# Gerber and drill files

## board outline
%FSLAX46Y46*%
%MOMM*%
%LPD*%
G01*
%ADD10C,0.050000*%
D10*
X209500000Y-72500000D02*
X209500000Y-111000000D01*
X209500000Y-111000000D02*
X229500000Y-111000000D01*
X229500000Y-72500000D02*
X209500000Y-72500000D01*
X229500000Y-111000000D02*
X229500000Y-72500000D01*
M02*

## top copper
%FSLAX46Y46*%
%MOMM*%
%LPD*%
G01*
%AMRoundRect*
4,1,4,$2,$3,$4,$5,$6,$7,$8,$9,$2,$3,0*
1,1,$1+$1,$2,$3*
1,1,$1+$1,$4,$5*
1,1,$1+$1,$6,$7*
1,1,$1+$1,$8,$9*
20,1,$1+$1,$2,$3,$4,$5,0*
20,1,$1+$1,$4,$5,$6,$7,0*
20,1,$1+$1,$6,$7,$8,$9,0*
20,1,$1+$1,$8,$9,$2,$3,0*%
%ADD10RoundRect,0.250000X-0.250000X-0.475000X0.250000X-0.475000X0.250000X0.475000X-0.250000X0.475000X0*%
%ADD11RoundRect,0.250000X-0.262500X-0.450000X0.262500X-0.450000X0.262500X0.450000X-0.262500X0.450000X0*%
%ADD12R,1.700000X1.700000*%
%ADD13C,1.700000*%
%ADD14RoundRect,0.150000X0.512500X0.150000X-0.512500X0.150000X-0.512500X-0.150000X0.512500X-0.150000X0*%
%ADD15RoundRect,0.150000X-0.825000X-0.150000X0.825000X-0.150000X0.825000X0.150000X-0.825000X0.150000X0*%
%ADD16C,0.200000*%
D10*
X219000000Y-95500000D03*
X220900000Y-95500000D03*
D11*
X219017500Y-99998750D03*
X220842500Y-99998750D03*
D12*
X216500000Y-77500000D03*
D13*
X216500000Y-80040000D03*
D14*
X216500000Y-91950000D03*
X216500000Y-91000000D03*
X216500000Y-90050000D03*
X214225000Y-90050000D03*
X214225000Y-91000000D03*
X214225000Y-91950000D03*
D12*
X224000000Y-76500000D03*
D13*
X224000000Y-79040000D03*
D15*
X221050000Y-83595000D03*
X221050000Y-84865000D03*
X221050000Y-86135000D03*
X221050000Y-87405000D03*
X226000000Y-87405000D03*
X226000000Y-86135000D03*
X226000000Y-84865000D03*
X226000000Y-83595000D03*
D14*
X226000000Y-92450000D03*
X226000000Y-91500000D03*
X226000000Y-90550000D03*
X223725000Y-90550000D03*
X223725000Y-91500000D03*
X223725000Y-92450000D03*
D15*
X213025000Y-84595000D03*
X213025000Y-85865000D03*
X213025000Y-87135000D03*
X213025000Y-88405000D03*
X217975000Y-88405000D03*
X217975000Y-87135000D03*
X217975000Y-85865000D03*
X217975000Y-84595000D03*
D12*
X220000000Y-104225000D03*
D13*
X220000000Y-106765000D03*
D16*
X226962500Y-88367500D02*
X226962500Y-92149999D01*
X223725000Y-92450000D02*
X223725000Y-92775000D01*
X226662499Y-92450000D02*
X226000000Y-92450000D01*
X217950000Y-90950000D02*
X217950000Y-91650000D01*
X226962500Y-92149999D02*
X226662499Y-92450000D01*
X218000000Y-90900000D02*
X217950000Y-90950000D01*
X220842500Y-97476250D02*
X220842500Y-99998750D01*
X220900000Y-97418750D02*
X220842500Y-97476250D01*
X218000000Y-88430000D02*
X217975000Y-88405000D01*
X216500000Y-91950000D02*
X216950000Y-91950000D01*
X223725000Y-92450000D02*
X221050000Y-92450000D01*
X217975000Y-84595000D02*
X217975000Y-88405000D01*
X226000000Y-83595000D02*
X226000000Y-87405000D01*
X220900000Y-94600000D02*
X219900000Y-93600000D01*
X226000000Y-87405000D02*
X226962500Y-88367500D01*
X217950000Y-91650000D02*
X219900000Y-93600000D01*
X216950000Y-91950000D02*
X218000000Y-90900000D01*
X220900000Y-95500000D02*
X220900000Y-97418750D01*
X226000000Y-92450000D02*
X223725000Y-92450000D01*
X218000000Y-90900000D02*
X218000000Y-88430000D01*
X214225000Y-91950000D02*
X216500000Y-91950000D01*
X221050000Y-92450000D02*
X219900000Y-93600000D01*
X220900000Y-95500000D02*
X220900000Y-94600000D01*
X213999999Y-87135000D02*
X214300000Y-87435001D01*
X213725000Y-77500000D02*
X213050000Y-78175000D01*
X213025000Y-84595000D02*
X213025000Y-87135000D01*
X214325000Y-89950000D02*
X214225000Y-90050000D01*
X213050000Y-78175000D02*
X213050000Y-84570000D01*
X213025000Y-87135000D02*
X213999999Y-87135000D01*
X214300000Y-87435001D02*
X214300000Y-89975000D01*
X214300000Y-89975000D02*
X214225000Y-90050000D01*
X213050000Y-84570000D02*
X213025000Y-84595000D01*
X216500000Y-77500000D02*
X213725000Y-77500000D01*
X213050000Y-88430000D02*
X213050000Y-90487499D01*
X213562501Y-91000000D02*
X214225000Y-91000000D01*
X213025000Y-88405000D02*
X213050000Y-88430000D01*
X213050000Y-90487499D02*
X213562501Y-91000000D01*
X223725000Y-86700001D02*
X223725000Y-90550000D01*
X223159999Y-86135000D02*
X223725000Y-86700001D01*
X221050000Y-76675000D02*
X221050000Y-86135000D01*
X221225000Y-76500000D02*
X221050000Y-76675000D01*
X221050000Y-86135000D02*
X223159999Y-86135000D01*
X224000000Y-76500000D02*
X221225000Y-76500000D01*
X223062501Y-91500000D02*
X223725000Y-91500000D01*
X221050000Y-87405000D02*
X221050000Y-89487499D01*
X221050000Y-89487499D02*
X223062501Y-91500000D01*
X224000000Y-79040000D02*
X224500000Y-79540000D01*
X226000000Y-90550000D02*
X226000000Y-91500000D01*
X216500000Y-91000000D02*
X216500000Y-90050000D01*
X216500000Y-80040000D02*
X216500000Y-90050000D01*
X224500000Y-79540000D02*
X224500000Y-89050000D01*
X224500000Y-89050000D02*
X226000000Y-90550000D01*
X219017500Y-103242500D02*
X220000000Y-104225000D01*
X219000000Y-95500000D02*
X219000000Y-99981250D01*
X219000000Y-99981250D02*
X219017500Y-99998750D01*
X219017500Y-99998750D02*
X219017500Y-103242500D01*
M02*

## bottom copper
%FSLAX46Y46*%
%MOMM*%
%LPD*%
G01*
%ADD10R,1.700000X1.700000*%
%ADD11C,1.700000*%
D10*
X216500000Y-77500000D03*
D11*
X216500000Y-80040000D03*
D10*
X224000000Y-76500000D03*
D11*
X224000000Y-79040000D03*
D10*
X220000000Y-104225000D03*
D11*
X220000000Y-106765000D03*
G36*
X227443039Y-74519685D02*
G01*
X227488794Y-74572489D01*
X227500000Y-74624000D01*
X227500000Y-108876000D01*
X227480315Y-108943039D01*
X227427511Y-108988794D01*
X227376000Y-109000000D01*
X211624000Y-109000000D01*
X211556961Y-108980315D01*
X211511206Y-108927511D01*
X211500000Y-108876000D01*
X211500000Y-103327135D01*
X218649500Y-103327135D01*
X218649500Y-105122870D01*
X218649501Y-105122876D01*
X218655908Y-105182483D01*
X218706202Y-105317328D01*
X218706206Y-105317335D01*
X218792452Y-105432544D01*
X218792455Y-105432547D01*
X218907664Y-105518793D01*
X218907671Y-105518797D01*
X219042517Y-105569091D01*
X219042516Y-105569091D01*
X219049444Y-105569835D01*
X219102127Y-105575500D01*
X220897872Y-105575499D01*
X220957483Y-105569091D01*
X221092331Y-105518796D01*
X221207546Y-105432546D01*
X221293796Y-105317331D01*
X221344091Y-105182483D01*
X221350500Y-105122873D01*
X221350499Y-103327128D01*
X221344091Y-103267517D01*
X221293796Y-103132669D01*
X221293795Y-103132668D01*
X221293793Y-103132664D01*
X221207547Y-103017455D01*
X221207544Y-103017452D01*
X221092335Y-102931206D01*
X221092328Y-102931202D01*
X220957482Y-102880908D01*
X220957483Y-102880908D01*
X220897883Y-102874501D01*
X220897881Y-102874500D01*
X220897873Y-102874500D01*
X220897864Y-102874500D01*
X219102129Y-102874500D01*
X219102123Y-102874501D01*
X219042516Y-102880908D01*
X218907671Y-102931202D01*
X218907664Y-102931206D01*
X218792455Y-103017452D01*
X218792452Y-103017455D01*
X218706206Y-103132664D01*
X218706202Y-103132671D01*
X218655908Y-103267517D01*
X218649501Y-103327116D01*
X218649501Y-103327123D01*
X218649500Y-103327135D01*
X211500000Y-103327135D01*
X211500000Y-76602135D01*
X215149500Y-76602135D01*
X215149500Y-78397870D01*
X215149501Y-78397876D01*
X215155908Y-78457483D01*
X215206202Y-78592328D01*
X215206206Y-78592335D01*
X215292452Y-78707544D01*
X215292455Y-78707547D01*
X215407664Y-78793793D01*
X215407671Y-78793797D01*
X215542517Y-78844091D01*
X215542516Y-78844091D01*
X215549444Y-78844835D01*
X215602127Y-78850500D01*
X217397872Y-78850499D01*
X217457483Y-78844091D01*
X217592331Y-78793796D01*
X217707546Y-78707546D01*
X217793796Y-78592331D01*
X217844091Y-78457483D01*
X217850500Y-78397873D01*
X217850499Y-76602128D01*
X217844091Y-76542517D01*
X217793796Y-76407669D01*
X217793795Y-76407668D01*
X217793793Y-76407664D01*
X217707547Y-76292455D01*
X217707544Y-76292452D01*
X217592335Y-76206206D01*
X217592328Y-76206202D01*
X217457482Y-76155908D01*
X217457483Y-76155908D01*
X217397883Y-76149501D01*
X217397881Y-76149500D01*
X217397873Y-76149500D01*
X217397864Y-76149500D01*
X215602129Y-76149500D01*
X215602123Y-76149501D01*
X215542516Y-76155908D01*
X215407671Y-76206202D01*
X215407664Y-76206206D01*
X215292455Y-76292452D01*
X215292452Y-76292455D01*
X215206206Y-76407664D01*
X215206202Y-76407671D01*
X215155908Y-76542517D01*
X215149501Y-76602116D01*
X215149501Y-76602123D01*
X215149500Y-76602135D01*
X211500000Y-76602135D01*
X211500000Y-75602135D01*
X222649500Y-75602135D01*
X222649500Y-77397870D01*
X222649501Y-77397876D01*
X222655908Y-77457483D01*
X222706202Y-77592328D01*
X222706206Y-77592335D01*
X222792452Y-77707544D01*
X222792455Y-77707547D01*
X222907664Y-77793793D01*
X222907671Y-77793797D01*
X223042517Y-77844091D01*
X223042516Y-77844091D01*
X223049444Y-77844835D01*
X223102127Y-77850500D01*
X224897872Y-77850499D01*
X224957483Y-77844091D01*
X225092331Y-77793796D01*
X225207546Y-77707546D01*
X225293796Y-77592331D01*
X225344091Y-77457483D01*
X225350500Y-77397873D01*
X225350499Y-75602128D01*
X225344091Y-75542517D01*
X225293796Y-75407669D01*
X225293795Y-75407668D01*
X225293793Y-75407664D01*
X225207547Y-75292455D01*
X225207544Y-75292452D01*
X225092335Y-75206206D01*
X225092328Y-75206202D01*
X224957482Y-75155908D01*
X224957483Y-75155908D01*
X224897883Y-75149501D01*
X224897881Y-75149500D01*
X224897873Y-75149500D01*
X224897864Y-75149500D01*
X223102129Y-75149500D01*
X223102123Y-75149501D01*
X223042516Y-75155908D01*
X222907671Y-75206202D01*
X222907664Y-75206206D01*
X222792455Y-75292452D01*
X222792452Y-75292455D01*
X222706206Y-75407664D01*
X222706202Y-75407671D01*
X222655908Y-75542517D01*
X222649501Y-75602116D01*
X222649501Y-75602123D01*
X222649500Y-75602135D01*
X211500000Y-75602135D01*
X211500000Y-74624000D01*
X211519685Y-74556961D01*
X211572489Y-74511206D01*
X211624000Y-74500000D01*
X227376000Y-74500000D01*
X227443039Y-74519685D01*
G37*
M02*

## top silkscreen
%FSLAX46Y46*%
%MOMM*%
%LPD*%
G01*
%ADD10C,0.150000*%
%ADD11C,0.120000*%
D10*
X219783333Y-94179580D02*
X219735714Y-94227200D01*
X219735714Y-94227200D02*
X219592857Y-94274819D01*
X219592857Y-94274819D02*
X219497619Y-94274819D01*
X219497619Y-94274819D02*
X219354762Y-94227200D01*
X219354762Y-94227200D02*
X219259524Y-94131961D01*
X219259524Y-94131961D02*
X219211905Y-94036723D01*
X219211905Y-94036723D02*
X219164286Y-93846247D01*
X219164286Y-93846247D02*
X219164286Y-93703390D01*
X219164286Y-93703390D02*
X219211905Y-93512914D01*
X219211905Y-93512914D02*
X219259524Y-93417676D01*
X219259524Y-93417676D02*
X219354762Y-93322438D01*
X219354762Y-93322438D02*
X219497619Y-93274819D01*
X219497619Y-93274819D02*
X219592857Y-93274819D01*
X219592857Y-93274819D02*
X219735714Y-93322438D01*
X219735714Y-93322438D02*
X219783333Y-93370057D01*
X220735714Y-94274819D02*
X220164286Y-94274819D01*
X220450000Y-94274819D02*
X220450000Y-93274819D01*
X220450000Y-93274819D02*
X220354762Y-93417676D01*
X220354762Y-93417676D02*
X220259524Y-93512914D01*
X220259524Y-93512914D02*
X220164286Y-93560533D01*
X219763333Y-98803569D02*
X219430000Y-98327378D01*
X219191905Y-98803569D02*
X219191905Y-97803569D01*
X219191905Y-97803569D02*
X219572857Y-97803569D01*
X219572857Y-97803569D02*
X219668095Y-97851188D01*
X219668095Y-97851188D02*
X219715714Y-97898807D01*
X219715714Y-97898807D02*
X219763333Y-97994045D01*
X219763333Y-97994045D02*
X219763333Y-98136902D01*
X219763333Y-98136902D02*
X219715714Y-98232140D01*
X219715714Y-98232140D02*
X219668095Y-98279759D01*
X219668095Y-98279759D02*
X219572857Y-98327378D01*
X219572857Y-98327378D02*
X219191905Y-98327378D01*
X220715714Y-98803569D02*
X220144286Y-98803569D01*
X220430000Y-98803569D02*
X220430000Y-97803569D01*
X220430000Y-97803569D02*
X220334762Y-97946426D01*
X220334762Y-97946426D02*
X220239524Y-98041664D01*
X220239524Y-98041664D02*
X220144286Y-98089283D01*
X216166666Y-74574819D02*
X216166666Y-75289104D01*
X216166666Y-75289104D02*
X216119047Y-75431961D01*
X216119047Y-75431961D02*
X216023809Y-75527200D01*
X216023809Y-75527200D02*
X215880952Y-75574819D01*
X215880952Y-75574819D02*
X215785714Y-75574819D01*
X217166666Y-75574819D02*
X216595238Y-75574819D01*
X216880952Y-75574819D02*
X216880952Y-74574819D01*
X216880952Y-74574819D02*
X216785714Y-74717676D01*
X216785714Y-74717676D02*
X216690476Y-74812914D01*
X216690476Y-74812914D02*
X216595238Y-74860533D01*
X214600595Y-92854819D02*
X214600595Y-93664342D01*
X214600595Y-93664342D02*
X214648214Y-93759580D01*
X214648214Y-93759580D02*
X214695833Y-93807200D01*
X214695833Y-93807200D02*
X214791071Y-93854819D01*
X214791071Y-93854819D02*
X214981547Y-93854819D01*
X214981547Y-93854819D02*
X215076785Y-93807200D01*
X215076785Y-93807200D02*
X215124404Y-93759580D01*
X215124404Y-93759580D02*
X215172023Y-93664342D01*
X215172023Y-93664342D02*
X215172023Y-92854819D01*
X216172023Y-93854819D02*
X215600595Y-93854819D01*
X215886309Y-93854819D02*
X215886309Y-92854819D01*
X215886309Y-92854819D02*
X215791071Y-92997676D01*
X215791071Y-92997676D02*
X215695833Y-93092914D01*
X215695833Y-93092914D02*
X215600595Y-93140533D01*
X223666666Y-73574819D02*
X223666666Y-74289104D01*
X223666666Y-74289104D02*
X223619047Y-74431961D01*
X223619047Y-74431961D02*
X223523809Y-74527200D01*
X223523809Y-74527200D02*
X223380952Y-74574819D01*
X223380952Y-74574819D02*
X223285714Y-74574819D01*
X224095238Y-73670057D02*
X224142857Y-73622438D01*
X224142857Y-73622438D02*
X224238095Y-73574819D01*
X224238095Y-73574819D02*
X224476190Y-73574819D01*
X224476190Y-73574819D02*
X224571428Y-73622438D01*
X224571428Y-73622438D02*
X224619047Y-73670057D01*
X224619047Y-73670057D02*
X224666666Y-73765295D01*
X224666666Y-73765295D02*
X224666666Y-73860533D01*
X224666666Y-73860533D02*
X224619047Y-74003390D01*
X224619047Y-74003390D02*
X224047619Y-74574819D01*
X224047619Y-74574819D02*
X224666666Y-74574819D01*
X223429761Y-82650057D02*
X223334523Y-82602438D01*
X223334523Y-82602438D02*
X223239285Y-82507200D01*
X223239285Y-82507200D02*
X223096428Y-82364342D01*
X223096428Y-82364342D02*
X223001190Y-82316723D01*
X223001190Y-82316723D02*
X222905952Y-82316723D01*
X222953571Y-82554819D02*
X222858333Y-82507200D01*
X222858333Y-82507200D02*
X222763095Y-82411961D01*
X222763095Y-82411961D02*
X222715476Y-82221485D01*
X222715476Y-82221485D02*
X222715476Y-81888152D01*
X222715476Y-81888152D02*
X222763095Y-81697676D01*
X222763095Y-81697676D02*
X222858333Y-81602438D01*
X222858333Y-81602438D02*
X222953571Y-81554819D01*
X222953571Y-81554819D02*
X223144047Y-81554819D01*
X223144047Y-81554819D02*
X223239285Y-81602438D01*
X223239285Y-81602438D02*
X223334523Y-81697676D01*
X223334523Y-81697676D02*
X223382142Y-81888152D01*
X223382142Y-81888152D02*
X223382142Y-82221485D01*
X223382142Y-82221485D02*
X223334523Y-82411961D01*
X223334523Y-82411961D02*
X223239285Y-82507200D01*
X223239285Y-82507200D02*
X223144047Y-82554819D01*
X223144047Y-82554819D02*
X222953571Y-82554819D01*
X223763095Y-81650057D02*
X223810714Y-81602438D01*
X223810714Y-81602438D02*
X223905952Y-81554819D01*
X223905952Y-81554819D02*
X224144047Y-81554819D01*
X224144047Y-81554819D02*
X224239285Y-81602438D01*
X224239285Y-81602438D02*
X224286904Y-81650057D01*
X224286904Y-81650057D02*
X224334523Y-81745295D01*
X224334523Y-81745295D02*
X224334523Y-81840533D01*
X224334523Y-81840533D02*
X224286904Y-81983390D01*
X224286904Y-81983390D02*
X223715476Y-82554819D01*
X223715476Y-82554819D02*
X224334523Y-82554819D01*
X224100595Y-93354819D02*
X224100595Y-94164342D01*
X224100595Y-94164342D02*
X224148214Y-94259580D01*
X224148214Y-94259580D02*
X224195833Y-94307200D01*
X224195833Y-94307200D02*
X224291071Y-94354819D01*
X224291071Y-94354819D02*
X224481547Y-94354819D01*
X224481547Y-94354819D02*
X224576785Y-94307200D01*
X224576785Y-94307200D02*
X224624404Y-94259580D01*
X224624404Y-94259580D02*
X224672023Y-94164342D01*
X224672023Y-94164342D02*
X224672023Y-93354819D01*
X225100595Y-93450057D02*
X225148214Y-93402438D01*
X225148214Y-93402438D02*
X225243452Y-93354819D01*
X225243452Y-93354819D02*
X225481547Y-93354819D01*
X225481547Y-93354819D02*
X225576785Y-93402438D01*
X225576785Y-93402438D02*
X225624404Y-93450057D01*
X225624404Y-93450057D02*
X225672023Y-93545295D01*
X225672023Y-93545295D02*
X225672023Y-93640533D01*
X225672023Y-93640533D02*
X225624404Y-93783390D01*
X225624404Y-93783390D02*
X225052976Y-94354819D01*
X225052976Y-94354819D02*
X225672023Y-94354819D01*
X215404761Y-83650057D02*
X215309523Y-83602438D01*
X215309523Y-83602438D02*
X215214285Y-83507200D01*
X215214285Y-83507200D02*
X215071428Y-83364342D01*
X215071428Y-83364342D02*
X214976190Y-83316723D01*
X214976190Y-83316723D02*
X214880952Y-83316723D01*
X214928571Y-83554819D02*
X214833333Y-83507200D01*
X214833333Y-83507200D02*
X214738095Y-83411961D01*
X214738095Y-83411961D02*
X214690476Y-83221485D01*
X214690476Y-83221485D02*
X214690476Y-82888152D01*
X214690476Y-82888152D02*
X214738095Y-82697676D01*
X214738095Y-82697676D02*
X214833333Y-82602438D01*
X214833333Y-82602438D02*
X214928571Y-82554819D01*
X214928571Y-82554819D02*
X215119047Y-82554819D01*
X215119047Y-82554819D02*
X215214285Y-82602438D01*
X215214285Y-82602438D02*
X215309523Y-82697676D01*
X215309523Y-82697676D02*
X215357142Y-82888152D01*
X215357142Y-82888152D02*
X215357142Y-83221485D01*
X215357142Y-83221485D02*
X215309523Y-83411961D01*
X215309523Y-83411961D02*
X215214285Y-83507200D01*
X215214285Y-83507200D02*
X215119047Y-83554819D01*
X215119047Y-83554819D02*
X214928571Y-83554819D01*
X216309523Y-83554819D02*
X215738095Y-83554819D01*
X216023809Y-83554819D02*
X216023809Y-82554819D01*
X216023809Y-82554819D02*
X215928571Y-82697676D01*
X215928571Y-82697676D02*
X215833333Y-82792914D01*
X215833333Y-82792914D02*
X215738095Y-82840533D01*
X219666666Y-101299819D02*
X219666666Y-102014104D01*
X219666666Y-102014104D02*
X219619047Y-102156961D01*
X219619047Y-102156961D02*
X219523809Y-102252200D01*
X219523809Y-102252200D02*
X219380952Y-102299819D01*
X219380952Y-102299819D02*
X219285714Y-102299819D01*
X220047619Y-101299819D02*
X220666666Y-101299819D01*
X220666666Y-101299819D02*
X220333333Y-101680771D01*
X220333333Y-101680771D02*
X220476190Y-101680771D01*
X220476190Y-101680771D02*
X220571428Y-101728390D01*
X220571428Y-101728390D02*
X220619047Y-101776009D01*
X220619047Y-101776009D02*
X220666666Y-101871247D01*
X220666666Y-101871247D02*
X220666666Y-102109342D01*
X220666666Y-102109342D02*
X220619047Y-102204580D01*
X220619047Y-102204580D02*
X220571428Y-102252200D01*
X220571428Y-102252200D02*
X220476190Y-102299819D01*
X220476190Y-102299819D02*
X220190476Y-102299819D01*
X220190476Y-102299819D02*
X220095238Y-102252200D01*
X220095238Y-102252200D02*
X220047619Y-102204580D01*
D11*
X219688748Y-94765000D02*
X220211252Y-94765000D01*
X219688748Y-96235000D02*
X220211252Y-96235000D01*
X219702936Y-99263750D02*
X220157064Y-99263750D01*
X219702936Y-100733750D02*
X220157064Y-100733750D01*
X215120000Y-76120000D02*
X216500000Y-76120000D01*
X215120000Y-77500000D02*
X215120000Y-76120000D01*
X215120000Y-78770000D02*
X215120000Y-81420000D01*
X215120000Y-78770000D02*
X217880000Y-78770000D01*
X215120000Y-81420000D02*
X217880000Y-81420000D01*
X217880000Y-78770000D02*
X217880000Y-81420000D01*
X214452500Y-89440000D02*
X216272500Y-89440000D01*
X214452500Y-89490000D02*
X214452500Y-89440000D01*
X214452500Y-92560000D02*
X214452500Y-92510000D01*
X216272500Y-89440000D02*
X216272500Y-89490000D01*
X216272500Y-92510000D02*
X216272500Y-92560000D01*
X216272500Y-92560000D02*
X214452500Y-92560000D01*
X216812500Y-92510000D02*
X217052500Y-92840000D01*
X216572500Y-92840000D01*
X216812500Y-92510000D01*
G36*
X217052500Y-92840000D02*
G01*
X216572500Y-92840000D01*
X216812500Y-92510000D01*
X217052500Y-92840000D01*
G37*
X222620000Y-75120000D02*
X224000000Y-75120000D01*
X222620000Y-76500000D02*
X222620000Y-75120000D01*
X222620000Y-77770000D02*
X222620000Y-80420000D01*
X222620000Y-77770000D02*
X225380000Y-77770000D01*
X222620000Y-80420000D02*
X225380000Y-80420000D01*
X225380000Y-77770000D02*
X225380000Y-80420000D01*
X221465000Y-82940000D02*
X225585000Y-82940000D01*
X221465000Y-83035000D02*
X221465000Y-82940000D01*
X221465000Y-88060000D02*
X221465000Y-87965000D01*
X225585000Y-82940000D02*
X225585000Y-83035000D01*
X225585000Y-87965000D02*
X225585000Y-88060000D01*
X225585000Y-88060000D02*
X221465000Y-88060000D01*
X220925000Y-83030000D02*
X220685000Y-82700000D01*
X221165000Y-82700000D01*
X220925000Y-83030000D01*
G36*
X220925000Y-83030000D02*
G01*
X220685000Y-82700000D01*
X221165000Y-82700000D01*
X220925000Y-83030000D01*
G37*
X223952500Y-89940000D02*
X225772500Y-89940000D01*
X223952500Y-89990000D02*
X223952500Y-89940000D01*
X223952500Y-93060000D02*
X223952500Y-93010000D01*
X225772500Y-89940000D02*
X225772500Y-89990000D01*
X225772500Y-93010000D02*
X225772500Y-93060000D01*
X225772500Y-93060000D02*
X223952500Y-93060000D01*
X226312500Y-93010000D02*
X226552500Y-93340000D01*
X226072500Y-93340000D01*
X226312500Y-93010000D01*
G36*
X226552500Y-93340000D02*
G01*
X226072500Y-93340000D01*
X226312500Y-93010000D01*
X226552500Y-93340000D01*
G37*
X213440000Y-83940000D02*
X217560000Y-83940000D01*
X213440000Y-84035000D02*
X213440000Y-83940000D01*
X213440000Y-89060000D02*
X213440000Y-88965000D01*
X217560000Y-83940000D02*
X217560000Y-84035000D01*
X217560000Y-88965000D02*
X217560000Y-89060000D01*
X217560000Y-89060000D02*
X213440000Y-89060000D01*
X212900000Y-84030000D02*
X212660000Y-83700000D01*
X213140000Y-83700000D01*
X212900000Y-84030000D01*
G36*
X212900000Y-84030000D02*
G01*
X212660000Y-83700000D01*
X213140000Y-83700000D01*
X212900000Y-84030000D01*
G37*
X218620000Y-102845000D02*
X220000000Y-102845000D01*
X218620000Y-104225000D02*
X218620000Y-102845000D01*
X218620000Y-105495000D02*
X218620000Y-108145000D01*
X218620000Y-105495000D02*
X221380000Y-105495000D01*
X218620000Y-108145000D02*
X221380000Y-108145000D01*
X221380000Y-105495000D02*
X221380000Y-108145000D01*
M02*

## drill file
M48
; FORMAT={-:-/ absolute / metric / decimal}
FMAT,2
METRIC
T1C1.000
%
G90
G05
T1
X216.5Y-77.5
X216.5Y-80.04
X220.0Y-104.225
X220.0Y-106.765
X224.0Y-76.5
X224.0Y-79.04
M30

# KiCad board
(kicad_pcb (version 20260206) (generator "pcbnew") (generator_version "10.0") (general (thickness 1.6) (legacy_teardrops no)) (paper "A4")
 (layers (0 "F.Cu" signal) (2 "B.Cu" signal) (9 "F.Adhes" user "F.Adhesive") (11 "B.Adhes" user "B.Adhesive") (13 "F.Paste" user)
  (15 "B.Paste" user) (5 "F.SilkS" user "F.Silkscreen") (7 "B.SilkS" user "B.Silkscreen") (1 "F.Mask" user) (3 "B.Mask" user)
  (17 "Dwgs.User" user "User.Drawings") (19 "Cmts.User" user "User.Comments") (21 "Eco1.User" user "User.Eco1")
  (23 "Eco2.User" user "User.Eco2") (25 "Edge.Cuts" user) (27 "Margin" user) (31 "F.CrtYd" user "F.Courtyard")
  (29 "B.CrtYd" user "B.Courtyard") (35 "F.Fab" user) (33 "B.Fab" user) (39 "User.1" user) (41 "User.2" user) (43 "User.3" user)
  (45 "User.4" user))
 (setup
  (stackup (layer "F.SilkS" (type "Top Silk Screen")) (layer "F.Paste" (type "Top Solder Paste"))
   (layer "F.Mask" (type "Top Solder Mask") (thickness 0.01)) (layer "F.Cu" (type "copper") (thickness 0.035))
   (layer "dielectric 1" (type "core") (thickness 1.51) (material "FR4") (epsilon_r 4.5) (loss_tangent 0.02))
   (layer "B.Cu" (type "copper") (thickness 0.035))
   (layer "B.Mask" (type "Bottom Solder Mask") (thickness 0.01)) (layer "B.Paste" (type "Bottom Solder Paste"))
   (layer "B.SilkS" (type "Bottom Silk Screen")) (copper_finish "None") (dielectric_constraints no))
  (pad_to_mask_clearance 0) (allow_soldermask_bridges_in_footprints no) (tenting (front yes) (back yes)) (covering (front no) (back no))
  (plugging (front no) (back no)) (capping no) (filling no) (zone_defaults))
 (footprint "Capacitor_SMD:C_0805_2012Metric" (layer "F.Cu") (at 219.95 95.5)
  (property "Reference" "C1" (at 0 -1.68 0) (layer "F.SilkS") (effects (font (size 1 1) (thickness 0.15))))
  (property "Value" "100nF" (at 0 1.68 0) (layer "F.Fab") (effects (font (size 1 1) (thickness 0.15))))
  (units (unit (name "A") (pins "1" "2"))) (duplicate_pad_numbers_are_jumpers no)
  (fp_line (start -0.261252 -0.735) (end 0.261252 -0.735) (stroke (width 0.12) (type solid)) (layer "F.SilkS"))
  (fp_line (start -0.261252 0.735) (end 0.261252 0.735) (stroke (width 0.12) (type solid)) (layer "F.SilkS"))
  (pad "1" smd roundrect (at -0.95 0) (size 1 1.45) (layers "F.Cu" "F.Mask" "F.Paste") (roundrect_rratio 0.25) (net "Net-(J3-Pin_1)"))
  (pad "2" smd roundrect (at 0.95 0) (size 1 1.45) (layers "F.Cu" "F.Mask" "F.Paste") (roundrect_rratio 0.25) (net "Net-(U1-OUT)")))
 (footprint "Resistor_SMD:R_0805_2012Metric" (layer "F.Cu") (at 219.93 99.99875)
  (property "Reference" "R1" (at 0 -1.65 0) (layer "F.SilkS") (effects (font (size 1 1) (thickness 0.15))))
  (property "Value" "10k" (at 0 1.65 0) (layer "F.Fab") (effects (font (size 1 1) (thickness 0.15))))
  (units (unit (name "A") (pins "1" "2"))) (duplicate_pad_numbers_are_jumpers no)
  (fp_line (start -0.227064 -0.735) (end 0.227064 -0.735) (stroke (width 0.12) (type solid)) (layer "F.SilkS"))
  (fp_line (start -0.227064 0.735) (end 0.227064 0.735) (stroke (width 0.12) (type solid)) (layer "F.SilkS"))
  (pad "1" smd roundrect (at -0.9125 0) (size 1.025 1.4) (layers "F.Cu" "F.Mask" "F.Paste") (roundrect_rratio 0.243902)
   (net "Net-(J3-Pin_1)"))
  (pad "2" smd roundrect (at 0.9125 0) (size 1.025 1.4) (layers "F.Cu" "F.Mask" "F.Paste") (roundrect_rratio 0.243902) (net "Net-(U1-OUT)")))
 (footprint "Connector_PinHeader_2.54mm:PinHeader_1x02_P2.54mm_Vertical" (layer "F.Cu") (at 216.5 77.5)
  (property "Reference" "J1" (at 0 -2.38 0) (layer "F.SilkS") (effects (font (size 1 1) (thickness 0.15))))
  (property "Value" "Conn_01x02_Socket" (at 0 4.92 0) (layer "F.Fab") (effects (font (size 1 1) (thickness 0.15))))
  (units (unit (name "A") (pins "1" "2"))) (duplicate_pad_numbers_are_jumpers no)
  (fp_line (start -1.38 -1.38) (end 0 -1.38) (stroke (width 0.12) (type solid)) (layer "F.SilkS"))
  (fp_line (start -1.38 0) (end -1.38 -1.38) (stroke (width 0.12) (type solid)) (layer "F.SilkS"))
  (fp_line (start -1.38 1.27) (end -1.38 3.92) (stroke (width 0.12) (type solid)) (layer "F.SilkS"))
  (fp_line (start -1.38 1.27) (end 1.38 1.27) (stroke (width 0.12) (type solid)) (layer "F.SilkS"))
  (fp_line (start -1.38 3.92) (end 1.38 3.92) (stroke (width 0.12) (type solid)) (layer "F.SilkS"))
  (fp_line (start 1.38 1.27) (end 1.38 3.92) (stroke (width 0.12) (type solid)) (layer "F.SilkS"))
  (pad "1" thru_hole rect (at 0 0) (size 1.7 1.7) (drill 1) (layers "*.Cu" "*.Mask") (remove_unused_layers no) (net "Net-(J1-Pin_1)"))
  (pad "2" thru_hole circle (at 0 2.54) (size 1.7 1.7) (drill 1) (layers "*.Cu" "*.Mask") (remove_unused_layers no) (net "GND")))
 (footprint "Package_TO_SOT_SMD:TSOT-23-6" (layer "F.Cu") (at 215.3625 91 180)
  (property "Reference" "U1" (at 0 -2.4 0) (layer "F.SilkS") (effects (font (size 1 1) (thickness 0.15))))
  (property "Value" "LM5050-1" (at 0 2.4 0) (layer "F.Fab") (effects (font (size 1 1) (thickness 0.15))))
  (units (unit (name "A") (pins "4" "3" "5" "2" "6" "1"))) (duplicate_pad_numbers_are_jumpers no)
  (fp_line (start 0.91 1.56) (end -0.91 1.56) (stroke (width 0.12) (type solid)) (layer "F.SilkS"))
  (fp_line (start 0.91 1.51) (end 0.91 1.56) (stroke (width 0.12) (type solid)) (layer "F.SilkS"))
  (fp_line (start 0.91 -1.56) (end 0.91 -1.51) (stroke (width 0.12) (type solid)) (layer "F.SilkS"))
  (fp_line (start -0.91 1.56) (end -0.91 1.51) (stroke (width 0.12) (type solid)) (layer "F.SilkS"))
  (fp_line (start -0.91 -1.51) (end -0.91 -1.56) (stroke (width 0.12) (type solid)) (layer "F.SilkS"))
  (fp_line (start -0.91 -1.56) (end 0.91 -1.56) (stroke (width 0.12) (type solid)) (layer "F.SilkS"))
  (fp_poly (pts (xy -1.45 -1.51) (xy -1.69 -1.84) (xy -1.21 -1.84)) (stroke (width 0.12) (type solid)) (fill yes) (layer "F.SilkS"))
  (pad "1" smd roundrect (at -1.1375 -0.95 180) (size 1.325 0.6) (layers "F.Cu" "F.Mask" "F.Paste") (roundrect_rratio 0.25)
   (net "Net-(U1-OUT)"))
  (pad "2" smd roundrect (at -1.1375 0 180) (size 1.325 0.6) (layers "F.Cu" "F.Mask" "F.Paste") (roundrect_rratio 0.25) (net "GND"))
  (pad "3" smd roundrect (at -1.1375 0.95 180) (size 1.325 0.6) (layers "F.Cu" "F.Mask" "F.Paste") (roundrect_rratio 0.25) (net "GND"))
  (pad "4" smd roundrect (at 1.1375 0.95 180) (size 1.325 0.6) (layers "F.Cu" "F.Mask" "F.Paste") (roundrect_rratio 0.25)
   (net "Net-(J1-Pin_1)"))
  (pad "5" smd roundrect (at 1.1375 0 180) (size 1.325 0.6) (layers "F.Cu" "F.Mask" "F.Paste") (roundrect_rratio 0.25) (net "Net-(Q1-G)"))
  (pad "6" smd roundrect (at 1.1375 -0.95 180) (size 1.325 0.6) (layers "F.Cu" "F.Mask" "F.Paste") (roundrect_rratio 0.25)
   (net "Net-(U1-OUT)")))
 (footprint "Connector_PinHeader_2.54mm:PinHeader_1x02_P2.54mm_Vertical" (layer "F.Cu") (at 224 76.5)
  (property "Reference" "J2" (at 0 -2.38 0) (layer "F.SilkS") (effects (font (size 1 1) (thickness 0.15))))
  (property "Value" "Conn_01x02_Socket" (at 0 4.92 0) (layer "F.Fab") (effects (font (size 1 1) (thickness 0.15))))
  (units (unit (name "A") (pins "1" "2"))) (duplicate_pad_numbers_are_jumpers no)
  (fp_line (start -1.38 -1.38) (end 0 -1.38) (stroke (width 0.12) (type solid)) (layer "F.SilkS"))
  (fp_line (start -1.38 0) (end -1.38 -1.38) (stroke (width 0.12) (type solid)) (layer "F.SilkS"))
  (fp_line (start -1.38 1.27) (end -1.38 3.92) (stroke (width 0.12) (type solid)) (layer "F.SilkS"))
  (fp_line (start -1.38 1.27) (end 1.38 1.27) (stroke (width 0.12) (type solid)) (layer "F.SilkS"))
  (fp_line (start -1.38 3.92) (end 1.38 3.92) (stroke (width 0.12) (type solid)) (layer "F.SilkS"))
  (fp_line (start 1.38 1.27) (end 1.38 3.92) (stroke (width 0.12) (type solid)) (layer "F.SilkS"))
  (pad "1" thru_hole rect (at 0 0) (size 1.7 1.7) (drill 1) (layers "*.Cu" "*.Mask") (remove_unused_layers no) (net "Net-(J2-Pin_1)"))
  (pad "2" thru_hole circle (at 0 2.54) (size 1.7 1.7) (drill 1) (layers "*.Cu" "*.Mask") (remove_unused_layers no) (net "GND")))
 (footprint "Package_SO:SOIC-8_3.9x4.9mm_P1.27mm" (layer "F.Cu") (at 223.525 85.5)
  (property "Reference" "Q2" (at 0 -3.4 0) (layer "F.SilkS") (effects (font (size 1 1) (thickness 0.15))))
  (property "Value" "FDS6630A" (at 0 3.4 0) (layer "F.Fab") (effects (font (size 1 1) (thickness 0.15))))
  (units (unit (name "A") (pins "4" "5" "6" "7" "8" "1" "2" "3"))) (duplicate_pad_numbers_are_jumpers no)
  (fp_line (start -2.06 -2.56) (end 2.06 -2.56) (stroke (width 0.12) (type solid)) (layer "F.SilkS"))
  (fp_line (start -2.06 -2.465) (end -2.06 -2.56) (stroke (width 0.12) (type solid)) (layer "F.SilkS"))
  (fp_line (start -2.06 2.56) (end -2.06 2.465) (stroke (width 0.12) (type solid)) (layer "F.SilkS"))
  (fp_line (start 2.06 -2.56) (end 2.06 -2.465) (stroke (width 0.12) (type solid)) (layer "F.SilkS"))
  (fp_line (start 2.06 2.465) (end 2.06 2.56) (stroke (width 0.12) (type solid)) (layer "F.SilkS"))
  (fp_line (start 2.06 2.56) (end -2.06 2.56) (stroke (width 0.12) (type solid)) (layer "F.SilkS"))
  (fp_poly (pts (xy -2.6 -2.47) (xy -2.84 -2.8) (xy -2.36 -2.8)) (stroke (width 0.12) (type solid)) (fill yes) (layer "F.SilkS"))
  (pad "1" smd roundrect (at -2.475 -1.905) (size 1.95 0.6) (layers "F.Cu" "F.Mask" "F.Paste") (roundrect_rratio 0.25)
   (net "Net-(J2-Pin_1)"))
  (pad "2" smd roundrect (at -2.475 -0.635) (size 1.95 0.6) (layers "F.Cu" "F.Mask" "F.Paste") (roundrect_rratio 0.25)
   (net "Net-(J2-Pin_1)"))
  (pad "3" smd roundrect (at -2.475 0.635) (size 1.95 0.6) (layers "F.Cu" "F.Mask" "F.Paste") (roundrect_rratio 0.25) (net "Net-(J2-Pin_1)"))
  (pad "4" smd roundrect (at -2.475 1.905) (size 1.95 0.6) (layers "F.Cu" "F.Mask" "F.Paste") (roundrect_rratio 0.25) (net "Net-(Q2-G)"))
  (pad "5" smd roundrect (at 2.475 1.905) (size 1.95 0.6) (layers "F.Cu" "F.Mask" "F.Paste") (roundrect_rratio 0.25) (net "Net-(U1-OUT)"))
  (pad "6" smd roundrect (at 2.475 0.635) (size 1.95 0.6) (layers "F.Cu" "F.Mask" "F.Paste") (roundrect_rratio 0.25) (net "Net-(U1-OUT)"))
  (pad "7" smd roundrect (at 2.475 -0.635) (size 1.95 0.6) (layers "F.Cu" "F.Mask" "F.Paste") (roundrect_rratio 0.25) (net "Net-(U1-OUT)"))
  (pad "8" smd roundrect (at 2.475 -1.905) (size 1.95 0.6) (layers "F.Cu" "F.Mask" "F.Paste") (roundrect_rratio 0.25) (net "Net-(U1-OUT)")))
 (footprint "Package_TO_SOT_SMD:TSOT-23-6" (layer "F.Cu") (at 224.8625 91.5 180)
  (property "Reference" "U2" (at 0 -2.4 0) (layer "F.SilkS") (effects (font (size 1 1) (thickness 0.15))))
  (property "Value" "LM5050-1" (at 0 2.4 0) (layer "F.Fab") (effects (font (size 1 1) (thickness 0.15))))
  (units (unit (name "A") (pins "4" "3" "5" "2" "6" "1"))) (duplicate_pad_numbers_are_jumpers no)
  (fp_line (start 0.91 1.56) (end -0.91 1.56) (stroke (width 0.12) (type solid)) (layer "F.SilkS"))
  (fp_line (start 0.91 1.51) (end 0.91 1.56) (stroke (width 0.12) (type solid)) (layer "F.SilkS"))
  (fp_line (start 0.91 -1.56) (end 0.91 -1.51) (stroke (width 0.12) (type solid)) (layer "F.SilkS"))
  (fp_line (start -0.91 1.56) (end -0.91 1.51) (stroke (width 0.12) (type solid)) (layer "F.SilkS"))
  (fp_line (start -0.91 -1.51) (end -0.91 -1.56) (stroke (width 0.12) (type solid)) (layer "F.SilkS"))
  (fp_line (start -0.91 -1.56) (end 0.91 -1.56) (stroke (width 0.12) (type solid)) (layer "F.SilkS"))
  (fp_poly (pts (xy -1.45 -1.51) (xy -1.69 -1.84) (xy -1.21 -1.84)) (stroke (width 0.12) (type solid)) (fill yes) (layer "F.SilkS"))
  (pad "1" smd roundrect (at -1.1375 -0.95 180) (size 1.325 0.6) (layers "F.Cu" "F.Mask" "F.Paste") (roundrect_rratio 0.25)
   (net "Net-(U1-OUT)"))
  (pad "2" smd roundrect (at -1.1375 0 180) (size 1.325 0.6) (layers "F.Cu" "F.Mask" "F.Paste") (roundrect_rratio 0.25) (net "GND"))
  (pad "3" smd roundrect (at -1.1375 0.95 180) (size 1.325 0.6) (layers "F.Cu" "F.Mask" "F.Paste") (roundrect_rratio 0.25) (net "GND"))
  (pad "4" smd roundrect (at 1.1375 0.95 180) (size 1.325 0.6) (layers "F.Cu" "F.Mask" "F.Paste") (roundrect_rratio 0.25)
   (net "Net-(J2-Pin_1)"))
  (pad "5" smd roundrect (at 1.1375 0 180) (size 1.325 0.6) (layers "F.Cu" "F.Mask" "F.Paste") (roundrect_rratio 0.25) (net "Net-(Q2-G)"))
  (pad "6" smd roundrect (at 1.1375 -0.95 180) (size 1.325 0.6) (layers "F.Cu" "F.Mask" "F.Paste") (roundrect_rratio 0.25)
   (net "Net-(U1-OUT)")))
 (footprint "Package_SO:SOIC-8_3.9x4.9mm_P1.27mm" (layer "F.Cu") (at 215.5 86.5)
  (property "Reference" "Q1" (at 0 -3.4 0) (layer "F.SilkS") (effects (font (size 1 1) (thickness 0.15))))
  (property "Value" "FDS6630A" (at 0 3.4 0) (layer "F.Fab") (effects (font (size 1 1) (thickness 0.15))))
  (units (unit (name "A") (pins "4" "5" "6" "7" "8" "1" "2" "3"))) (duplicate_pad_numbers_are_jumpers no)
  (fp_line (start -2.06 -2.56) (end 2.06 -2.56) (stroke (width 0.12) (type solid)) (layer "F.SilkS"))
  (fp_line (start -2.06 -2.465) (end -2.06 -2.56) (stroke (width 0.12) (type solid)) (layer "F.SilkS"))
  (fp_line (start -2.06 2.56) (end -2.06 2.465) (stroke (width 0.12) (type solid)) (layer "F.SilkS"))
  (fp_line (start 2.06 -2.56) (end 2.06 -2.465) (stroke (width 0.12) (type solid)) (layer "F.SilkS"))
  (fp_line (start 2.06 2.465) (end 2.06 2.56) (stroke (width 0.12) (type solid)) (layer "F.SilkS"))
  (fp_line (start 2.06 2.56) (end -2.06 2.56) (stroke (width 0.12) (type solid)) (layer "F.SilkS"))
  (fp_poly (pts (xy -2.6 -2.47) (xy -2.84 -2.8) (xy -2.36 -2.8)) (stroke (width 0.12) (type solid)) (fill yes) (layer "F.SilkS"))
  (pad "1" smd roundrect (at -2.475 -1.905) (size 1.95 0.6) (layers "F.Cu" "F.Mask" "F.Paste") (roundrect_rratio 0.25)
   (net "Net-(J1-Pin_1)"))
  (pad "2" smd roundrect (at -2.475 -0.635) (size 1.95 0.6) (layers "F.Cu" "F.Mask" "F.Paste") (roundrect_rratio 0.25)
   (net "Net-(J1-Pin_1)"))
  (pad "3" smd roundrect (at -2.475 0.635) (size 1.95 0.6) (layers "F.Cu" "F.Mask" "F.Paste") (roundrect_rratio 0.25) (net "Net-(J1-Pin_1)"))
  (pad "4" smd roundrect (at -2.475 1.905) (size 1.95 0.6) (layers "F.Cu" "F.Mask" "F.Paste") (roundrect_rratio 0.25) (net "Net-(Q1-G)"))
  (pad "5" smd roundrect (at 2.475 1.905) (size 1.95 0.6) (layers "F.Cu" "F.Mask" "F.Paste") (roundrect_rratio 0.25) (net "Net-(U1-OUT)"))
  (pad "6" smd roundrect (at 2.475 0.635) (size 1.95 0.6) (layers "F.Cu" "F.Mask" "F.Paste") (roundrect_rratio 0.25) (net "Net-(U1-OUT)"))
  (pad "7" smd roundrect (at 2.475 -0.635) (size 1.95 0.6) (layers "F.Cu" "F.Mask" "F.Paste") (roundrect_rratio 0.25) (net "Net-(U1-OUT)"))
  (pad "8" smd roundrect (at 2.475 -1.905) (size 1.95 0.6) (layers "F.Cu" "F.Mask" "F.Paste") (roundrect_rratio 0.25) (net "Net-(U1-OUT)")))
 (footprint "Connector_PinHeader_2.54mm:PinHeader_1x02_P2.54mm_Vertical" (layer "F.Cu") (at 220 104.225)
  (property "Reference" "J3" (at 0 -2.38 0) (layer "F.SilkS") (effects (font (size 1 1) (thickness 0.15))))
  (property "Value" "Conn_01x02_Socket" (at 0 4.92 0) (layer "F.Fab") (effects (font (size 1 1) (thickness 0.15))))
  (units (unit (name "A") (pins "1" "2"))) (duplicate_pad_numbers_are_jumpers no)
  (fp_line (start -1.38 -1.38) (end 0 -1.38) (stroke (width 0.12) (type solid)) (layer "F.SilkS"))
  (fp_line (start -1.38 0) (end -1.38 -1.38) (stroke (width 0.12) (type solid)) (layer "F.SilkS"))
  (fp_line (start -1.38 1.27) (end -1.38 3.92) (stroke (width 0.12) (type solid)) (layer "F.SilkS"))
  (fp_line (start -1.38 1.27) (end 1.38 1.27) (stroke (width 0.12) (type solid)) (layer "F.SilkS"))
  (fp_line (start -1.38 3.92) (end 1.38 3.92) (stroke (width 0.12) (type solid)) (layer "F.SilkS"))
  (fp_line (start 1.38 1.27) (end 1.38 3.92) (stroke (width 0.12) (type solid)) (layer "F.SilkS"))
  (pad "1" thru_hole rect (at 0 0) (size 1.7 1.7) (drill 1) (layers "*.Cu" "*.Mask") (remove_unused_layers no) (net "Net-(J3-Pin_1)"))
  (pad "2" thru_hole circle (at 0 2.54) (size 1.7 1.7) (drill 1) (layers "*.Cu" "*.Mask") (remove_unused_layers no) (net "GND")))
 (gr_line (start 209.5 72.5) (end 209.5 111) (stroke (width 0.05) (type default)) (layer "Edge.Cuts"))
 (gr_line (start 209.5 111) (end 229.5 111) (stroke (width 0.05) (type default)) (layer "Edge.Cuts"))
 (gr_line (start 229.5 72.5) (end 209.5 72.5) (stroke (width 0.05) (type default)) (layer "Edge.Cuts"))
 (gr_line (start 229.5 111) (end 229.5 72.5) (stroke (width 0.05) (type default)) (layer "Edge.Cuts"))
 (segment (start 226.9625 88.3675) (end 226.9625 92.149999) (width 0.2) (layer "F.Cu") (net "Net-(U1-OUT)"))
 (segment (start 223.725 92.45) (end 223.725 92.775) (width 0.2) (layer "F.Cu") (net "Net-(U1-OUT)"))
 (segment (start 226.662499 92.45) (end 226 92.45) (width 0.2) (layer "F.Cu") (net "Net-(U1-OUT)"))
 (segment (start 217.95 90.95) (end 217.95 91.65) (width 0.2) (layer "F.Cu") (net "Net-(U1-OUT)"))
 (segment (start 226.9625 92.149999) (end 226.662499 92.45) (width 0.2) (layer "F.Cu") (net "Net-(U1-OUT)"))
 (segment (start 218 90.9) (end 217.95 90.95) (width 0.2) (layer "F.Cu") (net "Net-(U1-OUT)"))
 (segment (start 220.8425 97.47625) (end 220.8425 99.99875) (width 0.2) (layer "F.Cu") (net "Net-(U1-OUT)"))
 (segment (start 220.9 97.41875) (end 220.8425 97.47625) (width 0.2) (layer "F.Cu") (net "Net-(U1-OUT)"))
 (segment (start 218 88.43) (end 217.975 88.405) (width 0.2) (layer "F.Cu") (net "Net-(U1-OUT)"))
 (segment (start 216.5 91.95) (end 216.95 91.95) (width 0.2) (layer "F.Cu") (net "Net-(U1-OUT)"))
 (segment (start 223.725 92.45) (end 221.05 92.45) (width 0.2) (layer "F.Cu") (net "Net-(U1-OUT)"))
 (segment (start 217.975 84.595) (end 217.975 88.405) (width 0.2) (layer "F.Cu") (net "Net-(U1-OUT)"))
 (segment (start 226 83.595) (end 226 87.405) (width 0.2) (layer "F.Cu") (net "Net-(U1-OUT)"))
 (segment (start 220.9 94.6) (end 219.9 93.6) (width 0.2) (layer "F.Cu") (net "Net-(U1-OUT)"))
 (segment (start 226 87.405) (end 226.9625 88.3675) (width 0.2) (layer "F.Cu") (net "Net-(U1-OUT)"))
 (segment (start 217.95 91.65) (end 219.9 93.6) (width 0.2) (layer "F.Cu") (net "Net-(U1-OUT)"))
 (segment (start 216.95 91.95) (end 218 90.9) (width 0.2) (layer "F.Cu") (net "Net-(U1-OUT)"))
 (segment (start 220.9 95.5) (end 220.9 97.41875) (width 0.2) (layer "F.Cu") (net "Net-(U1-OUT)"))
 (segment (start 226 92.45) (end 223.725 92.45) (width 0.2) (layer "F.Cu") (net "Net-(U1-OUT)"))
 (segment (start 218 90.9) (end 218 88.43) (width 0.2) (layer "F.Cu") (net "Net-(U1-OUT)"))
 (segment (start 214.225 91.95) (end 216.5 91.95) (width 0.2) (layer "F.Cu") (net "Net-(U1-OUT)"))
 (segment (start 221.05 92.45) (end 219.9 93.6) (width 0.2) (layer "F.Cu") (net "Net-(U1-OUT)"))
 (segment (start 220.9 95.5) (end 220.9 94.6) (width 0.2) (layer "F.Cu") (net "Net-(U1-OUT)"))
 (segment (start 213.999999 87.135) (end 214.3 87.435001) (width 0.2) (layer "F.Cu") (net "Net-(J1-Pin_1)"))
 (segment (start 213.725 77.5) (end 213.05 78.175) (width 0.2) (layer "F.Cu") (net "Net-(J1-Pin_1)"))
 (segment (start 213.025 84.595) (end 213.025 87.135) (width 0.2) (layer "F.Cu") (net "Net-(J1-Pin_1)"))
 (segment (start 214.325 89.95) (end 214.225 90.05) (width 0.2) (layer "F.Cu") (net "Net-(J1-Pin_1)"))
 (segment (start 213.05 78.175) (end 213.05 84.57) (width 0.2) (layer "F.Cu") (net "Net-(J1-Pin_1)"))
 (segment (start 213.025 87.135) (end 213.999999 87.135) (width 0.2) (layer "F.Cu") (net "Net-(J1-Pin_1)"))
 (segment (start 214.3 87.435001) (end 214.3 89.975) (width 0.2) (layer "F.Cu") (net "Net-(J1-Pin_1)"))
 (segment (start 214.3 89.975) (end 214.225 90.05) (width 0.2) (layer "F.Cu") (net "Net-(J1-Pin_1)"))
 (segment (start 213.05 84.57) (end 213.025 84.595) (width 0.2) (layer "F.Cu") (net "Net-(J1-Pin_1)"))
 (segment (start 216.5 77.5) (end 213.725 77.5) (width 0.2) (layer "F.Cu") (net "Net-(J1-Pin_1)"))
 (segment (start 213.05 88.43) (end 213.05 90.487499) (width 0.2) (layer "F.Cu") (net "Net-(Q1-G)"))
 (segment (start 213.562501 91) (end 214.225 91) (width 0.2) (layer "F.Cu") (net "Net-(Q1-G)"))
 (segment (start 213.025 88.405) (end 213.05 88.43) (width 0.2) (layer "F.Cu") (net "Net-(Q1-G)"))
 (segment (start 213.05 90.487499) (end 213.562501 91) (width 0.2) (layer "F.Cu") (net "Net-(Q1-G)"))
 (segment (start 223.725 86.700001) (end 223.725 90.55) (width 0.2) (layer "F.Cu") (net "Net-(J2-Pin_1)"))
 (segment (start 223.159999 86.135) (end 223.725 86.700001) (width 0.2) (layer "F.Cu") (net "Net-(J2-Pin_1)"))
 (segment (start 221.05 76.675) (end 221.05 86.135) (width 0.2) (layer "F.Cu") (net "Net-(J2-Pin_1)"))
 (segment (start 221.225 76.5) (end 221.05 76.675) (width 0.2) (layer "F.Cu") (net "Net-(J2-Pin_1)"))
 (segment (start 221.05 86.135) (end 223.159999 86.135) (width 0.2) (layer "F.Cu") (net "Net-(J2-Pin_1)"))
 (segment (start 224 76.5) (end 221.225 76.5) (width 0.2) (layer "F.Cu") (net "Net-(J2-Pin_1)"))
 (segment (start 223.062501 91.5) (end 223.725 91.5) (width 0.2) (layer "F.Cu") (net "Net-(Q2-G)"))
 (segment (start 221.05 87.405) (end 221.05 89.487499) (width 0.2) (layer "F.Cu") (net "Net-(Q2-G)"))
 (segment (start 221.05 89.487499) (end 223.062501 91.5) (width 0.2) (layer "F.Cu") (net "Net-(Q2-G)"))
 (segment (start 224 79.04) (end 224.5 79.54) (width 0.2) (layer "F.Cu") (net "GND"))
 (segment (start 226 90.55) (end 226 91.5) (width 0.2) (layer "F.Cu") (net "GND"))
 (segment (start 216.5 91) (end 216.5 90.05) (width 0.2) (layer "F.Cu") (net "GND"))
 (segment (start 216.5 80.04) (end 216.5 90.05) (width 0.2) (layer "F.Cu") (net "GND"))
 (segment (start 224.5 79.54) (end 224.5 89.05) (width 0.2) (layer "F.Cu") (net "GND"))
 (segment (start 224.5 89.05) (end 226 90.55) (width 0.2) (layer "F.Cu") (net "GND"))
 (segment (start 219.0175 103.2425) (end 220 104.225) (width 0.2) (layer "F.Cu") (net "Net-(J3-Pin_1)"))
 (segment (start 219 95.5) (end 219 99.98125) (width 0.2) (layer "F.Cu") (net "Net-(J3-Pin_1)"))
 (segment (start 219 99.98125) (end 219.0175 99.99875) (width 0.2) (layer "F.Cu") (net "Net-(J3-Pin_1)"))
 (segment (start 219.0175 99.99875) (end 219.0175 103.2425) (width 0.2) (layer "F.Cu") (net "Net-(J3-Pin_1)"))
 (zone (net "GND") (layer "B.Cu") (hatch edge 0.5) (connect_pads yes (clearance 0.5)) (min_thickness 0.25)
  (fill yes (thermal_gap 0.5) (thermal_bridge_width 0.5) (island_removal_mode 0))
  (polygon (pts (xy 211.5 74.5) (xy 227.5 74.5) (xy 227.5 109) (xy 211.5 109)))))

